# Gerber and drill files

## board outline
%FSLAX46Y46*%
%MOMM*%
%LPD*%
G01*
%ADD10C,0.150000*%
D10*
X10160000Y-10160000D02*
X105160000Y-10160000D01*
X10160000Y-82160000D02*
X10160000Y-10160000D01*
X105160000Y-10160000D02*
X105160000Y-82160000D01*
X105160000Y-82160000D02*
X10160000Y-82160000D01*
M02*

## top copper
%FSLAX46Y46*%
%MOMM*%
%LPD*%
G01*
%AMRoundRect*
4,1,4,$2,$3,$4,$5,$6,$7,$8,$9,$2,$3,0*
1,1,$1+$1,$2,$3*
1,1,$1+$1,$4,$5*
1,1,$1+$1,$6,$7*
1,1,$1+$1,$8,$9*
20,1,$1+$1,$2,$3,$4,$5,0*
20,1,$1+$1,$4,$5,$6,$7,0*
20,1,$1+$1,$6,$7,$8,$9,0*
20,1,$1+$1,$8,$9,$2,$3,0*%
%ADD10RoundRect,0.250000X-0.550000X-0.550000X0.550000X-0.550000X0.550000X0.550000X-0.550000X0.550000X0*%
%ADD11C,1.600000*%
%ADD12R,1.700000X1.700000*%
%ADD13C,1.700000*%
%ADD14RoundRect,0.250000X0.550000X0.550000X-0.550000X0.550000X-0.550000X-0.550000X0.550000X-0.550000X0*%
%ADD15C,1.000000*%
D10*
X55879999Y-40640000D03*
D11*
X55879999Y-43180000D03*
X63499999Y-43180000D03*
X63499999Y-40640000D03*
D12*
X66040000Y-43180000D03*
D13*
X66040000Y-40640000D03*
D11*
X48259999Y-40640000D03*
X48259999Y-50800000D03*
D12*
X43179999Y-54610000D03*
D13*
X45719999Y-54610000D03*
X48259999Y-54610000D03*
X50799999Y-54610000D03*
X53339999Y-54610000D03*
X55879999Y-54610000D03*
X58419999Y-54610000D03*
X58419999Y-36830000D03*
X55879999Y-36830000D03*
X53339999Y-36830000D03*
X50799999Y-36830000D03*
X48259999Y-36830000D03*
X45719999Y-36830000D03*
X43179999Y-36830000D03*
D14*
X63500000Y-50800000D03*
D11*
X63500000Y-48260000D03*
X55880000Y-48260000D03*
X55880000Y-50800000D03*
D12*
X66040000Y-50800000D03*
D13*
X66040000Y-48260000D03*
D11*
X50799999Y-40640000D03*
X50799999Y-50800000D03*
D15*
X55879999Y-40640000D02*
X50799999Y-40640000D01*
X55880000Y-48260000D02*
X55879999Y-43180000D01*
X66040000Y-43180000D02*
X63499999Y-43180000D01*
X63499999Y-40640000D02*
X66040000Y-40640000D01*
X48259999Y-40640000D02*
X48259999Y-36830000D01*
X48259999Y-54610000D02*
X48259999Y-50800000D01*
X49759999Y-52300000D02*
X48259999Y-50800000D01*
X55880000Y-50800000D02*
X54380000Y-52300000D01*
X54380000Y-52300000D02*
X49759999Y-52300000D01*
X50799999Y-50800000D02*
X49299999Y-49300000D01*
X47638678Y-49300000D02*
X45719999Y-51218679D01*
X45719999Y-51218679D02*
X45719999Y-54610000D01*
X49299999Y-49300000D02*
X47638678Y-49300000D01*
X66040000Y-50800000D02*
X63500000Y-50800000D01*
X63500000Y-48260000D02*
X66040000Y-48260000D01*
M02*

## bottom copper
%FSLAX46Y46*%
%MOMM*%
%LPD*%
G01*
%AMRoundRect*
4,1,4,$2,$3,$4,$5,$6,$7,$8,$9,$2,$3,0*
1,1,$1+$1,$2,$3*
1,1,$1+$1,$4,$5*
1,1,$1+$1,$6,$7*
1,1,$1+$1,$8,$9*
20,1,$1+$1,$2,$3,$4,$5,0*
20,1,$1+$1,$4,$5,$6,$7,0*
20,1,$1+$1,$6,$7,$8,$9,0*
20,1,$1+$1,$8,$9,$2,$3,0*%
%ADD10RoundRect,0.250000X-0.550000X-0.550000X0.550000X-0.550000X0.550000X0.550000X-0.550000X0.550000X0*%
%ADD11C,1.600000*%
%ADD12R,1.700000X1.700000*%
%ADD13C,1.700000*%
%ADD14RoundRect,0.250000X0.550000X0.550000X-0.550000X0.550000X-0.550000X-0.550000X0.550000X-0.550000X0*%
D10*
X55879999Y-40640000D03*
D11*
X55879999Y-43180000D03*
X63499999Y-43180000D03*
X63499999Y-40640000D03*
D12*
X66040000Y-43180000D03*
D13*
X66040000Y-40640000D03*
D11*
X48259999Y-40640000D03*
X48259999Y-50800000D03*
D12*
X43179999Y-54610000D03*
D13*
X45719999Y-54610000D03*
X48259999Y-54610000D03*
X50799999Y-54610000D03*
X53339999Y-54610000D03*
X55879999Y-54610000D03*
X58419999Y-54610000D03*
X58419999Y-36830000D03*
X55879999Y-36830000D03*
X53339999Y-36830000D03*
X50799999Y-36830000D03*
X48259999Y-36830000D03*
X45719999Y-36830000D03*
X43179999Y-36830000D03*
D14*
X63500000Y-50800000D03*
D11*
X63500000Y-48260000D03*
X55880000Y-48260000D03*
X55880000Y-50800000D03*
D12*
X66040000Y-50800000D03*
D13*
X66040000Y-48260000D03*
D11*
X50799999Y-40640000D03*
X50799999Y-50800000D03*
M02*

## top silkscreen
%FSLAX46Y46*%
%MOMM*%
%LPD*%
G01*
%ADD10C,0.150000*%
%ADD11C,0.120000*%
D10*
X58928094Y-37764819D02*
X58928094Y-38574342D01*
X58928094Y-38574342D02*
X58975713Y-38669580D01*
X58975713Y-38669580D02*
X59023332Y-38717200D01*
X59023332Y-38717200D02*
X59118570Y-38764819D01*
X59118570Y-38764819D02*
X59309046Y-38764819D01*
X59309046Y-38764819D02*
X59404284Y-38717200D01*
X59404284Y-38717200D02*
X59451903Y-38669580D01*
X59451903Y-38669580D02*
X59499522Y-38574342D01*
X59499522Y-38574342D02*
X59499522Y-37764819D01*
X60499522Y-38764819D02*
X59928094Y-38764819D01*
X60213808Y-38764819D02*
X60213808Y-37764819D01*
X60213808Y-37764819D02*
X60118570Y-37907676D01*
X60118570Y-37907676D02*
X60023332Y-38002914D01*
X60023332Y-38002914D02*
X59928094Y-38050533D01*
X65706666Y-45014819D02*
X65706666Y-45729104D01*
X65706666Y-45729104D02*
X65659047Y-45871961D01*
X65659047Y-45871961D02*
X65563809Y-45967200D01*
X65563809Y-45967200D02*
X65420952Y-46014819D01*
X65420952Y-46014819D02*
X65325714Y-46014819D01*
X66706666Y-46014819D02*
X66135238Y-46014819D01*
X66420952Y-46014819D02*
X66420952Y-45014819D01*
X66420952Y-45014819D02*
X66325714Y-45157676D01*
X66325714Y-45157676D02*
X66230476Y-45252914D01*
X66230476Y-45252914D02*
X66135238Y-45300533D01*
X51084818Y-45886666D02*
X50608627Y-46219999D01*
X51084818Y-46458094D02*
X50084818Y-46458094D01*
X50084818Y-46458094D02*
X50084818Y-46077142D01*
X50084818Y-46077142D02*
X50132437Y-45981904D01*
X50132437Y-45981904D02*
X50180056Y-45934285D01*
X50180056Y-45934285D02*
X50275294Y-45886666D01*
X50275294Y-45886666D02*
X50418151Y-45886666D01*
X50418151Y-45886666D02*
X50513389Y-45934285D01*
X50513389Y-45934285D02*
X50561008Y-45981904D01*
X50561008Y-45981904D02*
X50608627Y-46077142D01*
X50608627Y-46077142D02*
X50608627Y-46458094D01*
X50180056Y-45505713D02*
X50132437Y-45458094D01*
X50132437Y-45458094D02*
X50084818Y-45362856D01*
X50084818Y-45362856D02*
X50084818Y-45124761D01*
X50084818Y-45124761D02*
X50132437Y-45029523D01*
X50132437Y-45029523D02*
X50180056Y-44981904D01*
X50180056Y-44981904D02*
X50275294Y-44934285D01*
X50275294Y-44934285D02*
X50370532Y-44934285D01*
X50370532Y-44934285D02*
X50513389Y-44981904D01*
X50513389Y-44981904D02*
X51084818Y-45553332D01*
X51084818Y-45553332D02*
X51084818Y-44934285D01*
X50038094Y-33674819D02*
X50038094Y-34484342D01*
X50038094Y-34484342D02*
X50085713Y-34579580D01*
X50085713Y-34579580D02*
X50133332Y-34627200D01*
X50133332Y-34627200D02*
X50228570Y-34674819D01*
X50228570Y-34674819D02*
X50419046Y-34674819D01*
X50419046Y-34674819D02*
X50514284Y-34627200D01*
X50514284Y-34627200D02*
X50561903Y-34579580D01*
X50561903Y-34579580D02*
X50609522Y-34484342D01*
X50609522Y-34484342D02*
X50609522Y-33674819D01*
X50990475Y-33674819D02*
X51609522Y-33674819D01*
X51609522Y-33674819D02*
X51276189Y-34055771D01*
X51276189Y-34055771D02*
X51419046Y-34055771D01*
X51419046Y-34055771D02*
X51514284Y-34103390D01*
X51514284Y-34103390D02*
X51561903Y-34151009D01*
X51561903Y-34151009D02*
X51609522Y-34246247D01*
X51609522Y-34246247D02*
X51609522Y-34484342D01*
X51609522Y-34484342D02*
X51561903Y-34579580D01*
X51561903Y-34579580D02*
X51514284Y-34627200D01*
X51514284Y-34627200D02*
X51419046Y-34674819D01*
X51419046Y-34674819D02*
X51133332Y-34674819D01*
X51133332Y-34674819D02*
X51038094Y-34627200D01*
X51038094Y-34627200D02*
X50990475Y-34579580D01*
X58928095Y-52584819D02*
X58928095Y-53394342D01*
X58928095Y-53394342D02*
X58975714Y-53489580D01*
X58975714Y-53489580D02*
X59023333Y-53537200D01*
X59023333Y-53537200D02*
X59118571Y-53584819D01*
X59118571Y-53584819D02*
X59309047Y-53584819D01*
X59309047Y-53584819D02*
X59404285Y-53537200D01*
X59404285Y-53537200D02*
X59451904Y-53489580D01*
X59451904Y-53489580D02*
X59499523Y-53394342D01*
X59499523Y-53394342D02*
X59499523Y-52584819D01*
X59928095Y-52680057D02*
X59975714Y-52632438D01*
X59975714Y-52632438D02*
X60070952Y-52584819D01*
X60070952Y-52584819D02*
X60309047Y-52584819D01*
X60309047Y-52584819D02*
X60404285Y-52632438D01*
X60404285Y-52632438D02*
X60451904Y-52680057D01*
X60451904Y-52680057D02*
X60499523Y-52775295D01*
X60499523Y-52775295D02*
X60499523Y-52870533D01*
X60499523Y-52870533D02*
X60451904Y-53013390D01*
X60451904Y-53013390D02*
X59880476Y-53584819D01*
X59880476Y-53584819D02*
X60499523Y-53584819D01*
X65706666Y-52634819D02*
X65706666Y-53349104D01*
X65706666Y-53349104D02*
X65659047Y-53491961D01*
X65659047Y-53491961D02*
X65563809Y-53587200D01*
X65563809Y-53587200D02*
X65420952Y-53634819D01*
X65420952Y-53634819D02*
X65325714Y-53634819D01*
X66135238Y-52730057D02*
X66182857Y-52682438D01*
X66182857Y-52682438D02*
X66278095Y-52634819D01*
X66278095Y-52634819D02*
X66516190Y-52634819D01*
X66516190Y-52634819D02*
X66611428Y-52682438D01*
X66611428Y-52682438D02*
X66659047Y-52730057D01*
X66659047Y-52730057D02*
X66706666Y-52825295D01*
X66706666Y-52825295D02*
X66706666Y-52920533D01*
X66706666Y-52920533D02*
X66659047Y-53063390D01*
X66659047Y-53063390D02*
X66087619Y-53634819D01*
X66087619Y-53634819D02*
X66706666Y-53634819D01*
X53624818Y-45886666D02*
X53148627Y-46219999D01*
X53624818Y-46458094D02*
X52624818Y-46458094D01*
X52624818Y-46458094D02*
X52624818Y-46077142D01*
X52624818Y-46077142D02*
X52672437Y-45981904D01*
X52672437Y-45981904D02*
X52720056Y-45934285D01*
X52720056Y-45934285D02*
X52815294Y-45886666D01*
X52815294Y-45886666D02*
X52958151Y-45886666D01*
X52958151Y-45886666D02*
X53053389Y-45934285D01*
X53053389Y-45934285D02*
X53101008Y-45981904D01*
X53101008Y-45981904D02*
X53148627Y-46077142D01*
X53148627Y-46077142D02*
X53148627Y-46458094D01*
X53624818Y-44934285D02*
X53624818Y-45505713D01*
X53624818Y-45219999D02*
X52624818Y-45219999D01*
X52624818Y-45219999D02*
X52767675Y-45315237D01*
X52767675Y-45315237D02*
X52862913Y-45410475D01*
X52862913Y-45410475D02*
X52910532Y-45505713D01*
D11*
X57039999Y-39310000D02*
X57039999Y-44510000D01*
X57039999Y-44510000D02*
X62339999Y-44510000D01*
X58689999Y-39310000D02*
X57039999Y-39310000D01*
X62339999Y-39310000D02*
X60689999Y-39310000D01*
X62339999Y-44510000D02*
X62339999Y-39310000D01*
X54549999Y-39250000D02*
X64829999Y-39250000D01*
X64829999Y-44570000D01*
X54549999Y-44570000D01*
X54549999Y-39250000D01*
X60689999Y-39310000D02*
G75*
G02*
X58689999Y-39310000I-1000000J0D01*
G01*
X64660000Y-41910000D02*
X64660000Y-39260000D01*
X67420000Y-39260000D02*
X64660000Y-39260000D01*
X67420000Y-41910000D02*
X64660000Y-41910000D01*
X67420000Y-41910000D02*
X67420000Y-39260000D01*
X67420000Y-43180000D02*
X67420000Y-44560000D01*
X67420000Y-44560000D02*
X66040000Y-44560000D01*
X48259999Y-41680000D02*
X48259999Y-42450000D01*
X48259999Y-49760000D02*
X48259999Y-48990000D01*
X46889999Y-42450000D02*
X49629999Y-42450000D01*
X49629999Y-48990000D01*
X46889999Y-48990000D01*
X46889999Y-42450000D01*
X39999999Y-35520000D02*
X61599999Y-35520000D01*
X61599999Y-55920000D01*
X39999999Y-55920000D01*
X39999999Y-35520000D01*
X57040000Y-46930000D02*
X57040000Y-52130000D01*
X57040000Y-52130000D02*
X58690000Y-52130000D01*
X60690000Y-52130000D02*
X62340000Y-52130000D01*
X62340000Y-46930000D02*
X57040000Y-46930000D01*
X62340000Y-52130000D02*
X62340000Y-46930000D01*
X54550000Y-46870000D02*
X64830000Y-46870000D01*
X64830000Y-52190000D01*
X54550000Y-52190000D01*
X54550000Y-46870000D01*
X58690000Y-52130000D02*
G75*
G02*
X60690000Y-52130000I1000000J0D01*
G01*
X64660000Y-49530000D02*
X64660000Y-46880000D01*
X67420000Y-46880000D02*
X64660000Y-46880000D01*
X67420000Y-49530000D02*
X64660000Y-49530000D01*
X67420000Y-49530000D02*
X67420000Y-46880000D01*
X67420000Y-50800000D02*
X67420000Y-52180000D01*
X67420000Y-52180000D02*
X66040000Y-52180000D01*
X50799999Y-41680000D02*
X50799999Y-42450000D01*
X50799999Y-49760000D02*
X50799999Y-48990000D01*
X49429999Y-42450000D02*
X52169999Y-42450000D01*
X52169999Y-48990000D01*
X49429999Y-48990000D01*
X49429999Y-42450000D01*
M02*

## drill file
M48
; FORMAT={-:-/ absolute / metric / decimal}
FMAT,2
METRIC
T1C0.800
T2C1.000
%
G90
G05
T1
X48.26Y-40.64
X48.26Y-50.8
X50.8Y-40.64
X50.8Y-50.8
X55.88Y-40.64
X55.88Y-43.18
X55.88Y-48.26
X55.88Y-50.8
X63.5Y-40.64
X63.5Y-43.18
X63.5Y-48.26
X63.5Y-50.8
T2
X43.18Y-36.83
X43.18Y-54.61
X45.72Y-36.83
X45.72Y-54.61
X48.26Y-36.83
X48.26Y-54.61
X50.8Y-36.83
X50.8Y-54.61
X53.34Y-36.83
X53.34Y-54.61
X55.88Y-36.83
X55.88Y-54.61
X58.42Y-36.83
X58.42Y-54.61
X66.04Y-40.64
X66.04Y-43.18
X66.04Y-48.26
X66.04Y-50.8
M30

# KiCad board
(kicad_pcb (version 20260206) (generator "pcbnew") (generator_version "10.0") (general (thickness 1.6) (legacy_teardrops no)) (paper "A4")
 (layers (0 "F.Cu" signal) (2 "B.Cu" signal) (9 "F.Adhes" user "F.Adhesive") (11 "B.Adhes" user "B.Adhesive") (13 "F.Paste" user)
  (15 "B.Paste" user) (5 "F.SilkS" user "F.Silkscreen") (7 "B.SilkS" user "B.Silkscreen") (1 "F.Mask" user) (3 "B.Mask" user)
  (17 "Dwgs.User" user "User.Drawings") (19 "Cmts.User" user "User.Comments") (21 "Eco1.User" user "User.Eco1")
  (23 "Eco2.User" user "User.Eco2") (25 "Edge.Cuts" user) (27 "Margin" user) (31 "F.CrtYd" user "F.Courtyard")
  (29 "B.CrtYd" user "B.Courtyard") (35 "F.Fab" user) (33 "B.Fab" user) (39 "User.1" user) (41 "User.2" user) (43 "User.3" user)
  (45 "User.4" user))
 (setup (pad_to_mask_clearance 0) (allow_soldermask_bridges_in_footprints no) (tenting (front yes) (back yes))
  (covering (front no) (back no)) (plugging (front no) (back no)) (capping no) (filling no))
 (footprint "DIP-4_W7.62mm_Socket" (layer "F.Cu") (at 55.879999 40.64)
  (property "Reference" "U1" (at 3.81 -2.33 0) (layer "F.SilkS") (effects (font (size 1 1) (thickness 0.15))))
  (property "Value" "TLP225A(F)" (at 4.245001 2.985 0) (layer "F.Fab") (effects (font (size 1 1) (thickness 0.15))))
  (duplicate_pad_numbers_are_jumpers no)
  (fp_line (start 1.16 -1.33) (end 1.16 3.87) (stroke (width 0.12) (type solid)) (layer "F.SilkS"))
  (fp_line (start 1.16 3.87) (end 6.46 3.87) (stroke (width 0.12) (type solid)) (layer "F.SilkS"))
  (fp_line (start 2.81 -1.33) (end 1.16 -1.33) (stroke (width 0.12) (type solid)) (layer "F.SilkS"))
  (fp_line (start 6.46 -1.33) (end 4.81 -1.33) (stroke (width 0.12) (type solid)) (layer "F.SilkS"))
  (fp_line (start 6.46 3.87) (end 6.46 -1.33) (stroke (width 0.12) (type solid)) (layer "F.SilkS"))
  (fp_rect (start -1.33 -1.39) (end 8.95 3.93) (stroke (width 0.12) (type solid)) (fill no) (layer "F.SilkS"))
  (fp_arc (start 4.81 -1.33) (mid 3.81 -0.33) (end 2.81 -1.33) (stroke (width 0.12) (type solid)) (layer "F.SilkS"))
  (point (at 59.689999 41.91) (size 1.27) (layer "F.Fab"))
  (pad "1" thru_hole roundrect (at 0 0) (size 1.6 1.6) (drill 0.8) (layers "*.Cu" "*.Mask") (remove_unused_layers no)
   (roundrect_rratio 0.15625) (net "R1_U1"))
  (pad "2" thru_hole circle (at 0 2.54) (size 1.6 1.6) (drill 0.8) (layers "*.Cu" "*.Mask") (remove_unused_layers no) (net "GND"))
  (pad "3" thru_hole circle (at 7.62 2.54) (size 1.6 1.6) (drill 0.8) (layers "*.Cu" "*.Mask") (remove_unused_layers no) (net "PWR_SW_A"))
  (pad "4" thru_hole circle (at 7.62 0) (size 1.6 1.6) (drill 0.8) (layers "*.Cu" "*.Mask") (remove_unused_layers no) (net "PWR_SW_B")))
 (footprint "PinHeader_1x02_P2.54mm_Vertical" (layer "F.Cu") (at 66.04 43.18 180)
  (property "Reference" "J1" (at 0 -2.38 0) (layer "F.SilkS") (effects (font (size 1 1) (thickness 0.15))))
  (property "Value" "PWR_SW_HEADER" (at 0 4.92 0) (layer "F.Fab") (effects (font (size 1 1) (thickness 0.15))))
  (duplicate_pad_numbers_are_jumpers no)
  (fp_line (start 1.38 1.27) (end 1.38 3.92) (stroke (width 0.12) (type solid)) (layer "F.SilkS"))
  (fp_line (start -1.38 3.92) (end 1.38 3.92) (stroke (width 0.12) (type solid)) (layer "F.SilkS"))
  (fp_line (start -1.38 1.27) (end 1.38 1.27) (stroke (width 0.12) (type solid)) (layer "F.SilkS"))
  (fp_line (start -1.38 1.27) (end -1.38 3.92) (stroke (width 0.12) (type solid)) (layer "F.SilkS"))
  (fp_line (start -1.38 0) (end -1.38 -1.38) (stroke (width 0.12) (type solid)) (layer "F.SilkS"))
  (fp_line (start -1.38 -1.38) (end 0 -1.38) (stroke (width 0.12) (type solid)) (layer "F.SilkS"))
  (pad "1" thru_hole rect (at 0 0 180) (size 1.7 1.7) (drill 1) (layers "*.Cu" "*.Mask") (remove_unused_layers no) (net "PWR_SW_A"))
  (pad "2" thru_hole circle (at 0 2.54 180) (size 1.7 1.7) (drill 1) (layers "*.Cu" "*.Mask") (remove_unused_layers no) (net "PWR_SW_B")))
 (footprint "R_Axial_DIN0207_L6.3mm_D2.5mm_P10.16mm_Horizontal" (layer "F.Cu") (at 48.259999 40.64 -90)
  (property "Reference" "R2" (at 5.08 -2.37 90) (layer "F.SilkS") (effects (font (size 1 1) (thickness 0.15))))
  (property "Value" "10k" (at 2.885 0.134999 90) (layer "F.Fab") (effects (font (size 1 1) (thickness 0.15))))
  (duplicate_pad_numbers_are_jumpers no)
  (fp_line (start 1.04 0) (end 1.81 0) (stroke (width 0.12) (type solid)) (layer "F.SilkS"))
  (fp_line (start 9.12 0) (end 8.35 0) (stroke (width 0.12) (type solid)) (layer "F.SilkS"))
  (fp_rect (start 1.81 -1.37) (end 8.35 1.37) (stroke (width 0.12) (type solid)) (fill no) (layer "F.SilkS"))
  (pad "1" thru_hole circle (at 0 0 270) (size 1.6 1.6) (drill 0.8) (layers "*.Cu" "*.Mask") (remove_unused_layers no) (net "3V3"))
  (pad "2" thru_hole circle (at 10.16 0 270) (size 1.6 1.6) (drill 0.8) (layers "*.Cu" "*.Mask") (remove_unused_layers no) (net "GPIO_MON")))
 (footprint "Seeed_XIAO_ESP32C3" (layer "F.Cu") (at 50.799999 45.72)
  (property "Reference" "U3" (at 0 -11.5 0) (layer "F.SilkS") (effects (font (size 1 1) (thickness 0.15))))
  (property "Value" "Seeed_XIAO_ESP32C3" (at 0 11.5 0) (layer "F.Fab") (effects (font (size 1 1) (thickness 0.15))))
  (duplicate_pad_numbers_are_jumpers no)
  (fp_rect (start -10.8 -10.2) (end 10.8 10.2) (stroke (width 0.12) (type default)) (fill no) (layer "F.SilkS"))
  (pad "1" thru_hole rect (at -7.62 8.89) (size 1.7 1.7) (drill 1) (layers "*.Cu" "*.Mask") (remove_unused_layers no))
  (pad "2" thru_hole circle (at -5.08 8.89) (size 1.7 1.7) (drill 1) (layers "*.Cu" "*.Mask") (remove_unused_layers no) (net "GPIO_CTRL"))
  (pad "3" thru_hole circle (at -2.54 8.89) (size 1.7 1.7) (drill 1) (layers "*.Cu" "*.Mask") (remove_unused_layers no) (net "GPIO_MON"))
  (pad "4" thru_hole circle (at 0 8.89) (size 1.7 1.7) (drill 1) (layers "*.Cu" "*.Mask") (remove_unused_layers no))
  (pad "5" thru_hole circle (at 2.54 8.89) (size 1.7 1.7) (drill 1) (layers "*.Cu" "*.Mask") (remove_unused_layers no))
  (pad "6" thru_hole circle (at 5.08 8.89) (size 1.7 1.7) (drill 1) (layers "*.Cu" "*.Mask") (remove_unused_layers no))
  (pad "7" thru_hole circle (at 7.62 8.89) (size 1.7 1.7) (drill 1) (layers "*.Cu" "*.Mask") (remove_unused_layers no))
  (pad "8" thru_hole circle (at 7.62 -8.89) (size 1.7 1.7) (drill 1) (layers "*.Cu" "*.Mask") (remove_unused_layers no))
  (pad "9" thru_hole circle (at 5.08 -8.89) (size 1.7 1.7) (drill 1) (layers "*.Cu" "*.Mask") (remove_unused_layers no))
  (pad "10" thru_hole circle (at 2.54 -8.89) (size 1.7 1.7) (drill 1) (layers "*.Cu" "*.Mask") (remove_unused_layers no))
  (pad "11" thru_hole circle (at 0 -8.89) (size 1.7 1.7) (drill 1) (layers "*.Cu" "*.Mask") (remove_unused_layers no))
  (pad "12" thru_hole circle (at -2.54 -8.89) (size 1.7 1.7) (drill 1) (layers "*.Cu" "*.Mask") (remove_unused_layers no) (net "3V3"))
  (pad "13" thru_hole circle (at -5.08 -8.89) (size 1.7 1.7) (drill 1) (layers "*.Cu" "*.Mask") (remove_unused_layers no) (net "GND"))
  (pad "14" thru_hole circle (at -7.62 -8.89) (size 1.7 1.7) (drill 1) (layers "*.Cu" "*.Mask") (remove_unused_layers no)))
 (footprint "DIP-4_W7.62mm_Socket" (layer "F.Cu") (at 63.5 50.8 180)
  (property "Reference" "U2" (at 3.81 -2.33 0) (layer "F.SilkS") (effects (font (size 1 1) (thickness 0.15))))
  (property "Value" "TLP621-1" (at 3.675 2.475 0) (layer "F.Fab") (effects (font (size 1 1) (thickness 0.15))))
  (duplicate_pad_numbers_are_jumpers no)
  (fp_line (start 6.46 3.87) (end 6.46 -1.33) (stroke (width 0.12) (type solid)) (layer "F.SilkS"))
  (fp_line (start 6.46 -1.33) (end 4.81 -1.33) (stroke (width 0.12) (type solid)) (layer "F.SilkS"))
  (fp_line (start 2.81 -1.33) (end 1.16 -1.33) (stroke (width 0.12) (type solid)) (layer "F.SilkS"))
  (fp_line (start 1.16 3.87) (end 6.46 3.87) (stroke (width 0.12) (type solid)) (layer "F.SilkS"))
  (fp_line (start 1.16 -1.33) (end 1.16 3.87) (stroke (width 0.12) (type solid)) (layer "F.SilkS"))
  (fp_rect (start -1.33 -1.39) (end 8.95 3.93) (stroke (width 0.12) (type solid)) (fill no) (layer "F.SilkS"))
  (fp_arc (start 4.81 -1.33) (mid 3.81 -0.33) (end 2.81 -1.33) (stroke (width 0.12) (type solid)) (layer "F.SilkS"))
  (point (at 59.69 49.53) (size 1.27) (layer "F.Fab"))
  (pad "1" thru_hole roundrect (at 0 0 180) (size 1.6 1.6) (drill 0.8) (layers "*.Cu" "*.Mask") (remove_unused_layers no)
   (roundrect_rratio 0.15625) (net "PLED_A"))
  (pad "2" thru_hole circle (at 0 2.54 180) (size 1.6 1.6) (drill 0.8) (layers "*.Cu" "*.Mask") (remove_unused_layers no) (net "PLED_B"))
  (pad "3" thru_hole circle (at 7.62 2.54 180) (size 1.6 1.6) (drill 0.8) (layers "*.Cu" "*.Mask") (remove_unused_layers no) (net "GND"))
  (pad "4" thru_hole circle (at 7.62 0 180) (size 1.6 1.6) (drill 0.8) (layers "*.Cu" "*.Mask") (remove_unused_layers no) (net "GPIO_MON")))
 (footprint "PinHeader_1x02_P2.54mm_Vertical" (layer "F.Cu") (at 66.04 50.8 180)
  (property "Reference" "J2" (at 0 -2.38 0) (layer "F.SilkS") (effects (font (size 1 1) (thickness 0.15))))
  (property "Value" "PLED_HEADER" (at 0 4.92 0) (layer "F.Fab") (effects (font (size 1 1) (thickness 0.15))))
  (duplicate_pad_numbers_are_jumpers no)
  (fp_line (start 1.38 1.27) (end 1.38 3.92) (stroke (width 0.12) (type solid)) (layer "F.SilkS"))
  (fp_line (start -1.38 3.92) (end 1.38 3.92) (stroke (width 0.12) (type solid)) (layer "F.SilkS"))
  (fp_line (start -1.38 1.27) (end 1.38 1.27) (stroke (width 0.12) (type solid)) (layer "F.SilkS"))
  (fp_line (start -1.38 1.27) (end -1.38 3.92) (stroke (width 0.12) (type solid)) (layer "F.SilkS"))
  (fp_line (start -1.38 0) (end -1.38 -1.38) (stroke (width 0.12) (type solid)) (layer "F.SilkS"))
  (fp_line (start -1.38 -1.38) (end 0 -1.38) (stroke (width 0.12) (type solid)) (layer "F.SilkS"))
  (pad "1" thru_hole rect (at 0 0 180) (size 1.7 1.7) (drill 1) (layers "*.Cu" "*.Mask") (remove_unused_layers no) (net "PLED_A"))
  (pad "2" thru_hole circle (at 0 2.54 180) (size 1.7 1.7) (drill 1) (layers "*.Cu" "*.Mask") (remove_unused_layers no) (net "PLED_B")))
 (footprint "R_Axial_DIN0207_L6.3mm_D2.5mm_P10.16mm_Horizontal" (layer "F.Cu") (at 50.799999 40.64 -90)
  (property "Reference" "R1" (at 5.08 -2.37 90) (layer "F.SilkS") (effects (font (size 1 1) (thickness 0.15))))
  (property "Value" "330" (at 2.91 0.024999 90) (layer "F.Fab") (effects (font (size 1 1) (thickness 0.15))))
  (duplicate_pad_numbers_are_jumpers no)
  (fp_line (start 1.04 0) (end 1.81 0) (stroke (width 0.12) (type solid)) (layer "F.SilkS"))
  (fp_line (start 9.12 0) (end 8.35 0) (stroke (width 0.12) (type solid)) (layer "F.SilkS"))
  (fp_rect (start 1.81 -1.37) (end 8.35 1.37) (stroke (width 0.12) (type solid)) (fill no) (layer "F.SilkS"))
  (pad "1" thru_hole circle (at 0 0 270) (size 1.6 1.6) (drill 0.8) (layers "*.Cu" "*.Mask") (remove_unused_layers no) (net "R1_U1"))
  (pad "2" thru_hole circle (at 10.16 0 270) (size 1.6 1.6) (drill 0.8) (layers "*.Cu" "*.Mask") (remove_unused_layers no) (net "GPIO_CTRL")))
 (gr_line (start 10.16 10.16) (end 105.16 10.16) (stroke (width 0.15) (type default)) (layer "Edge.Cuts"))
 (gr_line (start 10.16 82.16) (end 10.16 10.16) (stroke (width 0.15) (type default)) (layer "Edge.Cuts"))
 (gr_line (start 105.16 10.16) (end 105.16 82.16) (stroke (width 0.15) (type default)) (layer "Edge.Cuts"))
 (gr_line (start 105.16 82.16) (end 10.16 82.16) (stroke (width 0.15) (type default)) (layer "Edge.Cuts"))
 (segment (start 55.879999 40.64) (end 50.799999 40.64) (width 1) (layer "F.Cu") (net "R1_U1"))
 (segment (start 55.88 48.26) (end 55.879999 43.18) (width 1) (layer "F.Cu") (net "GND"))
 (segment (start 66.04 43.18) (end 63.499999 43.18) (width 1) (layer "F.Cu") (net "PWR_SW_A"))
 (segment (start 63.499999 40.64) (end 66.04 40.64) (width 1) (layer "F.Cu") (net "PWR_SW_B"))
 (segment (start 48.259999 40.64) (end 48.259999 36.83) (width 1) (layer "F.Cu") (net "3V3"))
 (segment (start 48.259999 54.61) (end 48.259999 50.8) (width 1) (layer "F.Cu") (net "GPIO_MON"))
 (segment (start 49.759999 52.3) (end 48.259999 50.8) (width 1) (layer "F.Cu") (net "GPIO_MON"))
 (segment (start 55.88 50.8) (end 54.38 52.3) (width 1) (layer "F.Cu") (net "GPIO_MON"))
 (segment (start 54.38 52.3) (end 49.759999 52.3) (width 1) (layer "F.Cu") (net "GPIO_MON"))
 (segment (start 50.799999 50.8) (end 49.299999 49.3) (width 1) (layer "F.Cu") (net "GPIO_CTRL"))
 (segment (start 47.638678 49.3) (end 45.719999 51.218679) (width 1) (layer "F.Cu") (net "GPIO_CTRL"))
 (segment (start 45.719999 51.218679) (end 45.719999 54.61) (width 1) (layer "F.Cu") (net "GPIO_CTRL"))
 (segment (start 49.299999 49.3) (end 47.638678 49.3) (width 1) (layer "F.Cu") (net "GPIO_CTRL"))
 (segment (start 66.04 50.8) (end 63.5 50.8) (width 1) (layer "F.Cu") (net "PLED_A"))
 (segment (start 63.5 48.26) (end 66.04 48.26) (width 1) (layer "F.Cu") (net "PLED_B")))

